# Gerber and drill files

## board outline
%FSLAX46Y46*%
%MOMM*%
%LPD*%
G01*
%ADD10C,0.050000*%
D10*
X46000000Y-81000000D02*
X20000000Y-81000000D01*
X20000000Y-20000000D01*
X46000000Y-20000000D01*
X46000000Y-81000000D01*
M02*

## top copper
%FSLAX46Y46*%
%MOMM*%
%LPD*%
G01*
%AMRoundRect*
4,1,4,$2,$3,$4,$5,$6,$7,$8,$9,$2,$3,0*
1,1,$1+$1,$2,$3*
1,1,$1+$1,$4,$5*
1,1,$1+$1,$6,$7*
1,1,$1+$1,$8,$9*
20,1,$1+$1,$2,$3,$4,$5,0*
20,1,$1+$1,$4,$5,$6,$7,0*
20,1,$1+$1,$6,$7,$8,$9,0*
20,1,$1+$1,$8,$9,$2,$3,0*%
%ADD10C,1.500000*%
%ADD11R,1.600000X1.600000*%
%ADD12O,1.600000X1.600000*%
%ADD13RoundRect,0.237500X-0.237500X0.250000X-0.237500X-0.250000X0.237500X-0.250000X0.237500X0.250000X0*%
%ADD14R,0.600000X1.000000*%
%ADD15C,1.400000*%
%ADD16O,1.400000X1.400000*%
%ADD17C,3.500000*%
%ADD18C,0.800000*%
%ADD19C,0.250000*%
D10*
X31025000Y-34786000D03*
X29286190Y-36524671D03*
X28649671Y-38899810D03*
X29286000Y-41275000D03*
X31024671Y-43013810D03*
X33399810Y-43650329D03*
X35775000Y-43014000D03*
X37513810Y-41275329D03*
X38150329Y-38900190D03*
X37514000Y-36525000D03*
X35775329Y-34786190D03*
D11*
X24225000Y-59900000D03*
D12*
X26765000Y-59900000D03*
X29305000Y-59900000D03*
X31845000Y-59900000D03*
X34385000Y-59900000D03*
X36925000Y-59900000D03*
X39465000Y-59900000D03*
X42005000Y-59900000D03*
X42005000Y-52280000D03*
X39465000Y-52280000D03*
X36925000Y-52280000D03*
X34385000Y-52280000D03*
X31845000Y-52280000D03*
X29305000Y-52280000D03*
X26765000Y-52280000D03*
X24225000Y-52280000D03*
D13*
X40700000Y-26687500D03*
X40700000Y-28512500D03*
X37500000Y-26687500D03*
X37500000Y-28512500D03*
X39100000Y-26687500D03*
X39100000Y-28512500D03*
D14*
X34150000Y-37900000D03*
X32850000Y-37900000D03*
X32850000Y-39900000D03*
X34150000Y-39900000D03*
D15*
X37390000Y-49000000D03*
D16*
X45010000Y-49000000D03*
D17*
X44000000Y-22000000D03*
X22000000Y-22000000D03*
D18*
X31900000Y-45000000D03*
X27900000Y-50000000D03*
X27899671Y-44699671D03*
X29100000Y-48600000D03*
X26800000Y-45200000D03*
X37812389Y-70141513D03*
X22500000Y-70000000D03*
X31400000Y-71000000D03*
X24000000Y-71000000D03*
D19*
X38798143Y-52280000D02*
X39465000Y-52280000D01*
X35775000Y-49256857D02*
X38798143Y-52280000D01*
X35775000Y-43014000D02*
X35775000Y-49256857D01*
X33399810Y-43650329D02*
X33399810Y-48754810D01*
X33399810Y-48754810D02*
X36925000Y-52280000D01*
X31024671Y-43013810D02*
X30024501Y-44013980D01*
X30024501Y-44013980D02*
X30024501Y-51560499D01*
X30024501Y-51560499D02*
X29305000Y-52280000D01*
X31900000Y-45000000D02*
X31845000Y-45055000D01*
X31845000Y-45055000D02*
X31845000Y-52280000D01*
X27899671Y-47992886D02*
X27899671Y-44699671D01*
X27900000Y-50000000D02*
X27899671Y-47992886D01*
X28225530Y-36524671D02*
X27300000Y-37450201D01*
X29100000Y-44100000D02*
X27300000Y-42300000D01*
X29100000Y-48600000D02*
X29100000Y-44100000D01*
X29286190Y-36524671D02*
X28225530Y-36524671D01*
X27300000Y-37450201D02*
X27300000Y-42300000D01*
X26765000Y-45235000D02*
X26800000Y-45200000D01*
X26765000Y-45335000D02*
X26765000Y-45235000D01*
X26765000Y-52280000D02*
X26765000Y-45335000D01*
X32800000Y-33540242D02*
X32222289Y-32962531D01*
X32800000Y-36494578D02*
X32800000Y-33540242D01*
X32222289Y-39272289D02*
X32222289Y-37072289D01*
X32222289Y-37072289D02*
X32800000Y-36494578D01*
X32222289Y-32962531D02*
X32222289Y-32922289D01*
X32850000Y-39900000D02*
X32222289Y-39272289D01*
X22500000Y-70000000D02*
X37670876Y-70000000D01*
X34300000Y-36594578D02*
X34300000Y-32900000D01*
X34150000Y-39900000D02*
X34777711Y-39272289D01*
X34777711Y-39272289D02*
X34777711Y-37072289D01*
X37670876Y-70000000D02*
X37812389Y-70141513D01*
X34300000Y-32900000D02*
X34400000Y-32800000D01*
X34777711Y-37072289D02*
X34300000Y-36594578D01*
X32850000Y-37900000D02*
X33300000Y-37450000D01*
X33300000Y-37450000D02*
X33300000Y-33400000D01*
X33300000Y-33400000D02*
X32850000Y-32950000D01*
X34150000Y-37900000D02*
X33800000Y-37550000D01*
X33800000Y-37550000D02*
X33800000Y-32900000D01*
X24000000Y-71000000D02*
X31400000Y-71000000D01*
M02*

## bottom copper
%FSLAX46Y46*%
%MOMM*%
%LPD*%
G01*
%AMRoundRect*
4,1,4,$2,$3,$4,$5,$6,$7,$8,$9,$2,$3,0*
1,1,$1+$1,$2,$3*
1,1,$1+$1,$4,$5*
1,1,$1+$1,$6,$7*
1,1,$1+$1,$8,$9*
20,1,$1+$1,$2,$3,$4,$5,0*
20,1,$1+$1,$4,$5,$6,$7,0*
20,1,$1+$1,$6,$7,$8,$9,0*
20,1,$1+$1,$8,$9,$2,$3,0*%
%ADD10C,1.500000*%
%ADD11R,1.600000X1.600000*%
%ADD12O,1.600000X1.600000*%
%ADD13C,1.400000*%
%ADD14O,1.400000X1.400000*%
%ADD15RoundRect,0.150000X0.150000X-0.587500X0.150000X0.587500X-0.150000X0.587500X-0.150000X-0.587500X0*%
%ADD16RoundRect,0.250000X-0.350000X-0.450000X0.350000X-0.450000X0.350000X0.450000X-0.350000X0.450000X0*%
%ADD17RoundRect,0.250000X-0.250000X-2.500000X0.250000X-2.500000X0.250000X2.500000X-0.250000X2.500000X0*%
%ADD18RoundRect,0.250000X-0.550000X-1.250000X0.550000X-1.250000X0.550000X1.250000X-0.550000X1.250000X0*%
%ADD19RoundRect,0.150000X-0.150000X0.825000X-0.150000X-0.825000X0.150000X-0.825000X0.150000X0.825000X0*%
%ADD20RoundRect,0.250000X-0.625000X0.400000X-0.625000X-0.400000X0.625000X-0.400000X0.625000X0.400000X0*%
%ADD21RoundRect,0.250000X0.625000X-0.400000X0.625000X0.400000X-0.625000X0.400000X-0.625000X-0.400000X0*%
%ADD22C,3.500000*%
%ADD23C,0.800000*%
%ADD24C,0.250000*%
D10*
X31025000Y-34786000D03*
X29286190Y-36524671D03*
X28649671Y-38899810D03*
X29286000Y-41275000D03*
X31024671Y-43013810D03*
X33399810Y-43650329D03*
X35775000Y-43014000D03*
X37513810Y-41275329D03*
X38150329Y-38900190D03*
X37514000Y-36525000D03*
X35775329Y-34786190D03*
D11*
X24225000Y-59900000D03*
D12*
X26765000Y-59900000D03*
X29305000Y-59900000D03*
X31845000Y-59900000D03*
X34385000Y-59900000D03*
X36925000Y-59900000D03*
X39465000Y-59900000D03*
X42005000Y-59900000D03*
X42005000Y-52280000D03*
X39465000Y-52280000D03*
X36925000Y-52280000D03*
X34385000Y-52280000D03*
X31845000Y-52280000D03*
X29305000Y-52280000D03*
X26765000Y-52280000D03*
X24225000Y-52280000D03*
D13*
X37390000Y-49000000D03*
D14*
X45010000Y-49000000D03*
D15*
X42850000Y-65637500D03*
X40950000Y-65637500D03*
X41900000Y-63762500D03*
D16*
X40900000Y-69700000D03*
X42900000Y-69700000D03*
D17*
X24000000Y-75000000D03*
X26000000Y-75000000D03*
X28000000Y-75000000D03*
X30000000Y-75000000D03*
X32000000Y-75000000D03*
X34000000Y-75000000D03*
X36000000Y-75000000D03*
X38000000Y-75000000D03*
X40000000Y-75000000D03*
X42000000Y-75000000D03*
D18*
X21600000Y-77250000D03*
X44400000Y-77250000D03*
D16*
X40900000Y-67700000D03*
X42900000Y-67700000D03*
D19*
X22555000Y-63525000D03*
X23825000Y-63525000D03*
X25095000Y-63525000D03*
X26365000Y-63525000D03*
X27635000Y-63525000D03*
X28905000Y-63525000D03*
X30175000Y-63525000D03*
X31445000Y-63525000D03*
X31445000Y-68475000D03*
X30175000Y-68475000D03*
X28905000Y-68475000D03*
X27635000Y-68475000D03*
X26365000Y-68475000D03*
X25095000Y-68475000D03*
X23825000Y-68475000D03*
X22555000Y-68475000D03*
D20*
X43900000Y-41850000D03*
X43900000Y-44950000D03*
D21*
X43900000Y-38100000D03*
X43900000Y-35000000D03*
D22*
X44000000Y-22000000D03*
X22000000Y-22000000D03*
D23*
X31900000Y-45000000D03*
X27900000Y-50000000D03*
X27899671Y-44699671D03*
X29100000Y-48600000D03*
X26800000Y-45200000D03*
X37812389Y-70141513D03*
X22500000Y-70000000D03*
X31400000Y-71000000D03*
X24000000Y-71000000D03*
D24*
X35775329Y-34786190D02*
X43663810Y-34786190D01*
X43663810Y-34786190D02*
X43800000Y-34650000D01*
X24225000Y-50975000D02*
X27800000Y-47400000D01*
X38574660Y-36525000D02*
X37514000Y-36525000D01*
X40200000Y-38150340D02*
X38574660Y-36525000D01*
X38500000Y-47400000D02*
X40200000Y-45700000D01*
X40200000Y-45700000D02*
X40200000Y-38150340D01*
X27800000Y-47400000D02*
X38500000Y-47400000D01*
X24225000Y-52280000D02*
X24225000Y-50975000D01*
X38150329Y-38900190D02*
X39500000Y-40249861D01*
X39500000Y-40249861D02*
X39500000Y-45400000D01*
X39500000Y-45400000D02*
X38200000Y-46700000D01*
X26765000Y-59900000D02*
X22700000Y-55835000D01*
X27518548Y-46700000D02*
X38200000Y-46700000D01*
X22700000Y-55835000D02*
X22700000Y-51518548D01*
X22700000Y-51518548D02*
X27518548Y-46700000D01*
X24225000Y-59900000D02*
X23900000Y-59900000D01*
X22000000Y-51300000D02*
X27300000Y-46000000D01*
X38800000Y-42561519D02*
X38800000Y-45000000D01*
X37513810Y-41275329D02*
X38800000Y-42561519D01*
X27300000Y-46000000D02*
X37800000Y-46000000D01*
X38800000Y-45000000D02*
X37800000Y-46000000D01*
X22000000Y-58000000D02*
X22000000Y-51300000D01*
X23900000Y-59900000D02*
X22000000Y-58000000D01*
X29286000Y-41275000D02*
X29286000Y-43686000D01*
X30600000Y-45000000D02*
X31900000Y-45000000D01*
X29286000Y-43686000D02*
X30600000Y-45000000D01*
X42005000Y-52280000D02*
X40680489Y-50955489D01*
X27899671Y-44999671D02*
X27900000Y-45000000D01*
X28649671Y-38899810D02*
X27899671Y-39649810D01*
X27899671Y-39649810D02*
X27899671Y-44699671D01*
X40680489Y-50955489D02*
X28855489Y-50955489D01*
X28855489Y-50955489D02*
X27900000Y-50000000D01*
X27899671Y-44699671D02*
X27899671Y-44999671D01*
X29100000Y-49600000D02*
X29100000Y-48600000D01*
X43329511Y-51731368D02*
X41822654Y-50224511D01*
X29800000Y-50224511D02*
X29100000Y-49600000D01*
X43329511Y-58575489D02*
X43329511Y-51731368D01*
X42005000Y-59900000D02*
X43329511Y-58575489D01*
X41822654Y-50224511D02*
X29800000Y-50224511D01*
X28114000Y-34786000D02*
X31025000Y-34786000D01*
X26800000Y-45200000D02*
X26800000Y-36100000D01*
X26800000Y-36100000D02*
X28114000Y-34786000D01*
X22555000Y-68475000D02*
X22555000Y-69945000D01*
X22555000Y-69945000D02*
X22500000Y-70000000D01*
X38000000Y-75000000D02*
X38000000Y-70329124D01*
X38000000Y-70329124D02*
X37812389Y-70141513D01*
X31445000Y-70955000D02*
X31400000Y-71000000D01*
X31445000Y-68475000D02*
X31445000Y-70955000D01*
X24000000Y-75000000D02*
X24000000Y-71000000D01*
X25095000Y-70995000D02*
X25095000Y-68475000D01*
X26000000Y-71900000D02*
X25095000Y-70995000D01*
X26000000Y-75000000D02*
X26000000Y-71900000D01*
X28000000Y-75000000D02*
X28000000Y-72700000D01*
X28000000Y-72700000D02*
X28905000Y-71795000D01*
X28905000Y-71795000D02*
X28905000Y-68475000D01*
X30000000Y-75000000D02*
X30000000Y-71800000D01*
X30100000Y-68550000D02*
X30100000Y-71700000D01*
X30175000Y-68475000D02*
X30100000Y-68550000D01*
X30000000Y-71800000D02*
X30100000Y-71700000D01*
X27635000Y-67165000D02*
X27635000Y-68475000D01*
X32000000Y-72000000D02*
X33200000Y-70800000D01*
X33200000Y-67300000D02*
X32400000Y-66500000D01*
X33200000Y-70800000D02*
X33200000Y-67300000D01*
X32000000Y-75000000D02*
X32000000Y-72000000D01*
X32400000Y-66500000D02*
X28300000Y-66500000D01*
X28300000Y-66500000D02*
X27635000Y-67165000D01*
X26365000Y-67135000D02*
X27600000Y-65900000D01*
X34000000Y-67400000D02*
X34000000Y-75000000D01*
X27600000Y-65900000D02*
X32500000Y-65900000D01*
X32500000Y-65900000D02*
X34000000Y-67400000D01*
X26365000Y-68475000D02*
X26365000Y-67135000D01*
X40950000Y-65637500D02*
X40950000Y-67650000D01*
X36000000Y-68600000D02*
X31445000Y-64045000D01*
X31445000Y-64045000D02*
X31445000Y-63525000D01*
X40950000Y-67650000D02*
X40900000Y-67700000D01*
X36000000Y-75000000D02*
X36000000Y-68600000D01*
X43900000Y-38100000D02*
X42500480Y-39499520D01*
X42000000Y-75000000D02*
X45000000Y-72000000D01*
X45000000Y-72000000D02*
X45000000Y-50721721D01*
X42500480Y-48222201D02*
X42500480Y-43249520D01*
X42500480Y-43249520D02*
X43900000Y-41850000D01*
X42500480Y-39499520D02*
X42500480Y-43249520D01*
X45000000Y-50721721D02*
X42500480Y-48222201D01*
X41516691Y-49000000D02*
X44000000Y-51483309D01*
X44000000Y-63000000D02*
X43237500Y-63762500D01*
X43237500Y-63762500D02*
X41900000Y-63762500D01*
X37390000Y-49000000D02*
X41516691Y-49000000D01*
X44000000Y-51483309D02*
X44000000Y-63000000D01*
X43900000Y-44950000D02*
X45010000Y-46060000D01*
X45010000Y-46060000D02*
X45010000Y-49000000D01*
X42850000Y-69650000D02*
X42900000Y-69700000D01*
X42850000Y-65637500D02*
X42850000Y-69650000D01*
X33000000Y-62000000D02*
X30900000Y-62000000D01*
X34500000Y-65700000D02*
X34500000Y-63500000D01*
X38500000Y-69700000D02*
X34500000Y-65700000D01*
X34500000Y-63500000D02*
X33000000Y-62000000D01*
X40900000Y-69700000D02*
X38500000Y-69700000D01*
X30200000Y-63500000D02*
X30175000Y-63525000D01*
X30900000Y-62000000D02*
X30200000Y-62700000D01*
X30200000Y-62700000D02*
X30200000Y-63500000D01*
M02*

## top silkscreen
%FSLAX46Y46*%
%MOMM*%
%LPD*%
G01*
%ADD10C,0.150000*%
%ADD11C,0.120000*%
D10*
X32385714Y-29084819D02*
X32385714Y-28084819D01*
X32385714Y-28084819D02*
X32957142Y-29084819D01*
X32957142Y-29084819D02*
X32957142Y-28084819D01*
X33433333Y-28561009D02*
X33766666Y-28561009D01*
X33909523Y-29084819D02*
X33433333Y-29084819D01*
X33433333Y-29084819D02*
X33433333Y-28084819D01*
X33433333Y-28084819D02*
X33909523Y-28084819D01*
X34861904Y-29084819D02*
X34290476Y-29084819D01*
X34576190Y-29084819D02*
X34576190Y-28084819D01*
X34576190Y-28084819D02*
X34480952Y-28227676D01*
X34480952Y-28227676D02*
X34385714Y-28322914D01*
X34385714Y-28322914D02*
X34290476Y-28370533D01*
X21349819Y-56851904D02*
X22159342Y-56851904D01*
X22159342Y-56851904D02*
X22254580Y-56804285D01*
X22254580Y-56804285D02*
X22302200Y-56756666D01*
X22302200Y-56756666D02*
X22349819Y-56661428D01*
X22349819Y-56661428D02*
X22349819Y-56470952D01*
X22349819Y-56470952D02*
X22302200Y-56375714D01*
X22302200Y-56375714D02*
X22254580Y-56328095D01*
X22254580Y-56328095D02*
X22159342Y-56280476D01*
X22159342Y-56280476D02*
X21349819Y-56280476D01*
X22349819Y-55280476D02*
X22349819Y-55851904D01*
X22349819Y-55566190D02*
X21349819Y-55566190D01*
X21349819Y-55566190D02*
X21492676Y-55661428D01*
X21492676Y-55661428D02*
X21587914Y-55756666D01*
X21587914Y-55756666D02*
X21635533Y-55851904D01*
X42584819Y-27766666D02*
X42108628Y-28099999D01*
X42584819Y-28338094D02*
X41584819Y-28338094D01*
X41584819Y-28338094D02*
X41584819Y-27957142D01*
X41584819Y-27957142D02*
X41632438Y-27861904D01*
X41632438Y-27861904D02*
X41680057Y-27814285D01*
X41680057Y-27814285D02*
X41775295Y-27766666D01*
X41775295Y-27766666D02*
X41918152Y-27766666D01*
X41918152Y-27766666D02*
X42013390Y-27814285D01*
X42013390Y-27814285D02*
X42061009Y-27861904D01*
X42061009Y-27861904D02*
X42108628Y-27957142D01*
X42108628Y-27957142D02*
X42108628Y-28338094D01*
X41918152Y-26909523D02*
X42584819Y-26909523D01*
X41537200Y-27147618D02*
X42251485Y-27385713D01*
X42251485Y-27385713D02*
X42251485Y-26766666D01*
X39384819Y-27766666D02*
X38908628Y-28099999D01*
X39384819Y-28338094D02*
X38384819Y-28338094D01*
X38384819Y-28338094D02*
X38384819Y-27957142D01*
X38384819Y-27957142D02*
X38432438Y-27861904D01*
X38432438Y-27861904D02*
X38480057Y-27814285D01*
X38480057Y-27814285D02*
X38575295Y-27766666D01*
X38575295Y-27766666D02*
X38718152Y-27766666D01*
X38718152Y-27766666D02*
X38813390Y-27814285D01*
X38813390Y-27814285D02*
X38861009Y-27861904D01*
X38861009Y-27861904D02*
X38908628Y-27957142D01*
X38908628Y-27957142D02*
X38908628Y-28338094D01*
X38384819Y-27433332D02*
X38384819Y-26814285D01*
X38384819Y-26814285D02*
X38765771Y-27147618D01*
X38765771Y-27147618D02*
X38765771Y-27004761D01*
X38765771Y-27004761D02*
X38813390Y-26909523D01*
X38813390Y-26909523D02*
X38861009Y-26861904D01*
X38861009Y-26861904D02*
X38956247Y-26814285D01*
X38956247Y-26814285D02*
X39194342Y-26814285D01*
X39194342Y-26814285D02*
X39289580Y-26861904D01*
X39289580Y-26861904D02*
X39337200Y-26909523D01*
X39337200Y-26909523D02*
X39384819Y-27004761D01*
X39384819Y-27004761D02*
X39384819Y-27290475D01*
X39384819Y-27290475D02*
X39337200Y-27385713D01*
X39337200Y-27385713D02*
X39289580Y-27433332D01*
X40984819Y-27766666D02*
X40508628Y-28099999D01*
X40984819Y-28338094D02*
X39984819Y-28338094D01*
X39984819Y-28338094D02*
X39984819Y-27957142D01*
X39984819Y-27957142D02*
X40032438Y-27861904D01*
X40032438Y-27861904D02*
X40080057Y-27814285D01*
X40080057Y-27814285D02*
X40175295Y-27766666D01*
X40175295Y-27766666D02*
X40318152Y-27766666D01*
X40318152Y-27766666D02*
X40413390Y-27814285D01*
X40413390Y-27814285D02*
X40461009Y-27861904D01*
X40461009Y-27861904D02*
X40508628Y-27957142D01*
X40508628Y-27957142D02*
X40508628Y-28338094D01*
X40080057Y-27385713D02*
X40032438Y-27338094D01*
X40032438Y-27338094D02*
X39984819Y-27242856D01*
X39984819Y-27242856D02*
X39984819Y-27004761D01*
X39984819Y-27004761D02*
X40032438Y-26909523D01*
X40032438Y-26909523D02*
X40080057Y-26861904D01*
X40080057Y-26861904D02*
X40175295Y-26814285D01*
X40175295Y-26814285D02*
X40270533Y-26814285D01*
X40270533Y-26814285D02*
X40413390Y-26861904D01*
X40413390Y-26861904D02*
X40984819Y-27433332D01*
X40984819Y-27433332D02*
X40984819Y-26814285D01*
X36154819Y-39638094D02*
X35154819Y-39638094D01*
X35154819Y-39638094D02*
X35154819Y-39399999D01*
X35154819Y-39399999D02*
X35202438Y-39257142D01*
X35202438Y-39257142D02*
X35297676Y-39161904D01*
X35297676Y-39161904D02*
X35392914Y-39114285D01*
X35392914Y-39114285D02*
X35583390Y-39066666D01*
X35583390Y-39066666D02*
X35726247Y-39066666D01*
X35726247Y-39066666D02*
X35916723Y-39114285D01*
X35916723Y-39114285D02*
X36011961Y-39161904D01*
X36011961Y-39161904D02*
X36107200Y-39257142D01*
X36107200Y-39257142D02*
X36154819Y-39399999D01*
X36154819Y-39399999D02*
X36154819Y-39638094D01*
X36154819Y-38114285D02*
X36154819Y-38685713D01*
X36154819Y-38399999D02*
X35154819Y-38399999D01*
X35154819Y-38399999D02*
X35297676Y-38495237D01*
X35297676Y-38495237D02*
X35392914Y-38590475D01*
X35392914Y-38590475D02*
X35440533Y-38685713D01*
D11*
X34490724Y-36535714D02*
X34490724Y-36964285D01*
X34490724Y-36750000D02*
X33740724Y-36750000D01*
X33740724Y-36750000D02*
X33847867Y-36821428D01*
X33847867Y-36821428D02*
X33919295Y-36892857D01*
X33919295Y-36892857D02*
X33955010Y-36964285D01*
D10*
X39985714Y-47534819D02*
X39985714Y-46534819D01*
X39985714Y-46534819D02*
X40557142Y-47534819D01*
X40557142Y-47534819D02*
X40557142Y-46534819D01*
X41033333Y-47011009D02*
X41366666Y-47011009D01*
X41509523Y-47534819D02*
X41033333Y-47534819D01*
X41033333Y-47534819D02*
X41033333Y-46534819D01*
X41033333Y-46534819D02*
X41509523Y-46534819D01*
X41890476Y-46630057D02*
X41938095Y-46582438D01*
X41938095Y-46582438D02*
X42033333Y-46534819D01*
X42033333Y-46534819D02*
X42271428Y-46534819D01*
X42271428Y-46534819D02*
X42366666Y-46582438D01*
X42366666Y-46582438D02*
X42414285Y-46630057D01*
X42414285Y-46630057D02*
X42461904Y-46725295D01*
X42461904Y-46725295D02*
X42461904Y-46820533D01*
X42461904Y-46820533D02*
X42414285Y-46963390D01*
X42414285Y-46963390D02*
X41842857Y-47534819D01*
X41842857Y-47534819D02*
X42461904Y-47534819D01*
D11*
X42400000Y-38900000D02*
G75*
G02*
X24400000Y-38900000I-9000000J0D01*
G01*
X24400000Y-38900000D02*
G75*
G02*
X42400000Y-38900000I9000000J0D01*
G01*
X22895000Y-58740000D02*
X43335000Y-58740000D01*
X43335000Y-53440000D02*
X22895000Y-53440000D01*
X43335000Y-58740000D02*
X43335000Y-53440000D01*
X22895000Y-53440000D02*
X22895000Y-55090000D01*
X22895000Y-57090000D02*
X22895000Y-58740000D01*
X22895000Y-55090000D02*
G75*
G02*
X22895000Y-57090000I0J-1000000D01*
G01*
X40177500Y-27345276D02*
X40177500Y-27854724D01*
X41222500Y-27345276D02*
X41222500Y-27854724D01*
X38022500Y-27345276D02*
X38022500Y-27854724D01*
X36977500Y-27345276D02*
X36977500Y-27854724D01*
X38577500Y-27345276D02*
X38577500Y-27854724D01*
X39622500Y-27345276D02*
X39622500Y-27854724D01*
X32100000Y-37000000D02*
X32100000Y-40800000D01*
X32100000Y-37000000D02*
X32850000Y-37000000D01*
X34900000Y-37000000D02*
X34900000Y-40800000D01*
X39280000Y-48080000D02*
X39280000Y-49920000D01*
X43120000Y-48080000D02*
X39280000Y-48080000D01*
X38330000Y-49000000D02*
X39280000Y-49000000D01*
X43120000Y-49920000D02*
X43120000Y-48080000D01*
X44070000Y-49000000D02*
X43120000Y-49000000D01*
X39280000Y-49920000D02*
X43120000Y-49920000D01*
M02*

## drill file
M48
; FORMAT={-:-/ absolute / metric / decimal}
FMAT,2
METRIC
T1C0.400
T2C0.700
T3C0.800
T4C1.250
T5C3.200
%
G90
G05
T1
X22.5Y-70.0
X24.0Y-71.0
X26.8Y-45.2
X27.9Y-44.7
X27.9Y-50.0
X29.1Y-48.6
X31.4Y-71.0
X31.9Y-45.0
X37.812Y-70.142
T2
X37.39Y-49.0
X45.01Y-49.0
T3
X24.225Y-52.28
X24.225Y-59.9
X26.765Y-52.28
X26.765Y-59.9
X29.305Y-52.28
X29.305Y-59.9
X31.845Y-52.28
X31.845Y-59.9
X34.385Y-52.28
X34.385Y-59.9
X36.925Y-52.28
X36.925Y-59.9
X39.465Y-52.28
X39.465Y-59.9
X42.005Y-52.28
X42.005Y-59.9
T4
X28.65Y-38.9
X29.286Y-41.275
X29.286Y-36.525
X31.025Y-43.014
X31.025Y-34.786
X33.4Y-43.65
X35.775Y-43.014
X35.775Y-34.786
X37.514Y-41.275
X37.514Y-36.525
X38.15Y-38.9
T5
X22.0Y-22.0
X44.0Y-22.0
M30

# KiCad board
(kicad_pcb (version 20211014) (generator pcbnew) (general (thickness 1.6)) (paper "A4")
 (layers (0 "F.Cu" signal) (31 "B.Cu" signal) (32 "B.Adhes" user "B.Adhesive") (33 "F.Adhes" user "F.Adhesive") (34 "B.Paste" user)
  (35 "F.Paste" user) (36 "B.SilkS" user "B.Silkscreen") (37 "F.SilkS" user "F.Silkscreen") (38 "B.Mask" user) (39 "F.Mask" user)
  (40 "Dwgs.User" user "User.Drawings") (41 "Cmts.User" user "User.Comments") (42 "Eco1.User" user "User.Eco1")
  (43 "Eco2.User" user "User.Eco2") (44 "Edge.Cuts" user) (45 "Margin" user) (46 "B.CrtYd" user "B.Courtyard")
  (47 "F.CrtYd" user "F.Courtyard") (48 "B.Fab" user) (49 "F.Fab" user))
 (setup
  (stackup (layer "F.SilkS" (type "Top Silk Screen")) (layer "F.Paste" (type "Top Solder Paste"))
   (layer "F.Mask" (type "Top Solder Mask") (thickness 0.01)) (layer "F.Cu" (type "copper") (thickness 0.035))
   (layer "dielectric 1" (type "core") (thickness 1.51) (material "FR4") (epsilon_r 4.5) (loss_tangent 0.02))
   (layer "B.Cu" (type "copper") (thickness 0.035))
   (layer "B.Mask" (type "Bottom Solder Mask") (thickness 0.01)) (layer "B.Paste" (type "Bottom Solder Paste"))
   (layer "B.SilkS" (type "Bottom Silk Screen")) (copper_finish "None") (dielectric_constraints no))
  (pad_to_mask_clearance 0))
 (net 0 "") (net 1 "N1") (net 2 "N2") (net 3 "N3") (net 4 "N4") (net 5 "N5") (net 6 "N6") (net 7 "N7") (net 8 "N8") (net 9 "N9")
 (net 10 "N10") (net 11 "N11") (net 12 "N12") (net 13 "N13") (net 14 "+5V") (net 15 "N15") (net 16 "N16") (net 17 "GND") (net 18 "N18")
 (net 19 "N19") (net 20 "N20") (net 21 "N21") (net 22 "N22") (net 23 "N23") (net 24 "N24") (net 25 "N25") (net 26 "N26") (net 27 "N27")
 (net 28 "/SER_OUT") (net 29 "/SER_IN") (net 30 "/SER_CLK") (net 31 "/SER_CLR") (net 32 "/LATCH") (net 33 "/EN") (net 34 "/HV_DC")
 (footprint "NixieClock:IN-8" (layer "F.Cu") (at 33.5 38.9)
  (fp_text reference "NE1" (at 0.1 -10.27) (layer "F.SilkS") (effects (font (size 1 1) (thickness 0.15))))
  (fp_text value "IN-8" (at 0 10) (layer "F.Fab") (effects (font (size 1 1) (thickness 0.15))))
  (fp_circle (center -0.1 0) (end -0.1 9) (layer "F.SilkS") (width 0.12) (fill none))
  (pad "1" thru_hole circle locked (at -2.475 -4.114) (size 1.5 1.5) (drill 1.25) (layers *.Cu *.Mask) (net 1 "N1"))
  (pad "2" thru_hole circle locked (at -4.21381 -2.375329) (size 1.5 1.5) (drill 1.25) (layers *.Cu *.Mask) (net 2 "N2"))
  (pad "3" thru_hole circle locked (at -4.850329 -0.00019) (size 1.5 1.5) (drill 1.25) (layers *.Cu *.Mask) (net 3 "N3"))
  (pad "4" thru_hole circle locked (at -4.214 2.375) (size 1.5 1.5) (drill 1.25) (layers *.Cu *.Mask) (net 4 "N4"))
  (pad "5" thru_hole circle locked (at -2.475329 4.11381) (size 1.5 1.5) (drill 1.25) (layers *.Cu *.Mask) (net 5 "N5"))
  (pad "6" thru_hole circle locked (at -0.10019 4.750329) (size 1.5 1.5) (drill 1.25) (layers *.Cu *.Mask) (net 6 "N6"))
  (pad "7" thru_hole circle locked (at 2.275 4.114) (size 1.5 1.5) (drill 1.25) (layers *.Cu *.Mask) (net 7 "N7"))
  (pad "8" thru_hole circle locked (at 4.01381 2.375329) (size 1.5 1.5) (drill 1.25) (layers *.Cu *.Mask) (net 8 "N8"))
  (pad "9" thru_hole circle locked (at 4.650329 0.00019) (size 1.5 1.5) (drill 1.25) (layers *.Cu *.Mask) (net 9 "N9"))
  (pad "10" thru_hole circle locked (at 4.014 -2.375) (size 1.5 1.5) (drill 1.25) (layers *.Cu *.Mask) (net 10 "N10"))
  (pad "11" thru_hole circle locked (at 2.275329 -4.11381) (size 1.5 1.5) (drill 1.25) (layers *.Cu *.Mask) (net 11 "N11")))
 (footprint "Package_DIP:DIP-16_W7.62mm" (layer "F.Cu") (at 24.225 59.9 90)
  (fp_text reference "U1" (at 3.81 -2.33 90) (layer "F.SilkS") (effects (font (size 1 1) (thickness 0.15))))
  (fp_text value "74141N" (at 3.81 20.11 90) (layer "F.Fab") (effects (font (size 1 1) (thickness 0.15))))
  (fp_line (start 1.16 -1.33) (end 1.16 19.11) (layer "F.SilkS") (width 0.12))
  (fp_line (start 6.46 19.11) (end 6.46 -1.33) (layer "F.SilkS") (width 0.12))
  (fp_line (start 1.16 19.11) (end 6.46 19.11) (layer "F.SilkS") (width 0.12))
  (fp_line (start 6.46 -1.33) (end 4.81 -1.33) (layer "F.SilkS") (width 0.12))
  (fp_line (start 2.81 -1.33) (end 1.16 -1.33) (layer "F.SilkS") (width 0.12))
  (fp_arc (start 4.81 -1.33) (mid 3.81 -0.33) (end 2.81 -1.33) (layer "F.SilkS") (width 0.12))
  (pad "1" thru_hole rect locked (at 0 0 90) (size 1.6 1.6) (drill 0.8) (layers *.Cu *.Mask) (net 8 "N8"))
  (pad "2" thru_hole oval locked (at 0 2.54 90) (size 1.6 1.6) (drill 0.8) (layers *.Cu *.Mask) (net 9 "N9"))
  (pad "3" thru_hole oval locked (at 0 5.08 90) (size 1.6 1.6) (drill 0.8) (layers *.Cu *.Mask) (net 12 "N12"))
  (pad "4" thru_hole oval locked (at 0 7.62 90) (size 1.6 1.6) (drill 0.8) (layers *.Cu *.Mask) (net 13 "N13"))
  (pad "5" thru_hole oval locked (at 0 10.16 90) (size 1.6 1.6) (drill 0.8) (layers *.Cu *.Mask) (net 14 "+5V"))
  (pad "6" thru_hole oval locked (at 0 12.7 90) (size 1.6 1.6) (drill 0.8) (layers *.Cu *.Mask) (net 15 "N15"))
  (pad "7" thru_hole oval locked (at 0 15.24 90) (size 1.6 1.6) (drill 0.8) (layers *.Cu *.Mask) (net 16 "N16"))
  (pad "8" thru_hole oval locked (at 0 17.78 90) (size 1.6 1.6) (drill 0.8) (layers *.Cu *.Mask) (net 2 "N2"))
  (pad "9" thru_hole oval locked (at 7.62 17.78 90) (size 1.6 1.6) (drill 0.8) (layers *.Cu *.Mask) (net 3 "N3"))
  (pad "10" thru_hole oval locked (at 7.62 15.24 90) (size 1.6 1.6) (drill 0.8) (layers *.Cu *.Mask) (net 7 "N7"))
  (pad "11" thru_hole oval locked (at 7.62 12.7 90) (size 1.6 1.6) (drill 0.8) (layers *.Cu *.Mask) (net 6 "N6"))
  (pad "12" thru_hole oval locked (at 7.62 10.16 90) (size 1.6 1.6) (drill 0.8) (layers *.Cu *.Mask) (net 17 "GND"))
  (pad "13" thru_hole oval locked (at 7.62 7.62 90) (size 1.6 1.6) (drill 0.8) (layers *.Cu *.Mask) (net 4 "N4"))
  (pad "14" thru_hole oval locked (at 7.62 5.08 90) (size 1.6 1.6) (drill 0.8) (layers *.Cu *.Mask) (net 5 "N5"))
  (pad "15" thru_hole oval locked (at 7.62 2.54 90) (size 1.6 1.6) (drill 0.8) (layers *.Cu *.Mask) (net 1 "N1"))
  (pad "16" thru_hole oval locked (at 7.62 0 90) (size 1.6 1.6) (drill 0.8) (layers *.Cu *.Mask) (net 10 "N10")))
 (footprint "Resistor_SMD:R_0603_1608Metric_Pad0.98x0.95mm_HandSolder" (layer "F.Cu") (at 40.7 27.6 -90)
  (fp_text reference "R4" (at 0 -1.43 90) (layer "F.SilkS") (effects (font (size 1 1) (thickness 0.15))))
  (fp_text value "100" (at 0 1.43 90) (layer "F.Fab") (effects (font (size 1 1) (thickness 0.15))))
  (fp_line (start -0.254724 0.5225) (end 0.254724 0.5225) (layer "F.SilkS") (width 0.12))
  (fp_line (start -0.254724 -0.5225) (end 0.254724 -0.5225) (layer "F.SilkS") (width 0.12))
  (pad "1" smd roundrect locked (at -0.9125 0 270) (size 0.975 0.95) (layers "F.Cu" "F.Paste" "F.Mask") (roundrect_rratio 0.25)
   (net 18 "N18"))
  (pad "2" smd roundrect locked (at 0.9125 0 270) (size 0.975 0.95) (layers "F.Cu" "F.Paste" "F.Mask") (roundrect_rratio 0.25)
   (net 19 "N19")))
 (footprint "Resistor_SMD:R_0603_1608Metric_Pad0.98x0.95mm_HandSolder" (layer "F.Cu") (at 37.5 27.6 -90)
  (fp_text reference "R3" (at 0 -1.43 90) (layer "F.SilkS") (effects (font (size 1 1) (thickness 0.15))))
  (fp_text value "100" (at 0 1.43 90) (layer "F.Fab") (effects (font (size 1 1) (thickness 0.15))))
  (fp_line (start -0.254724 -0.5225) (end 0.254724 -0.5225) (layer "F.SilkS") (width 0.12))
  (fp_line (start -0.254724 0.5225) (end 0.254724 0.5225) (layer "F.SilkS") (width 0.12))
  (pad "1" smd roundrect locked (at -0.9125 0 270) (size 0.975 0.95) (layers "F.Cu" "F.Paste" "F.Mask") (roundrect_rratio 0.25)
   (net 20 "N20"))
  (pad "2" smd roundrect locked (at 0.9125 0 270) (size 0.975 0.95) (layers "F.Cu" "F.Paste" "F.Mask") (roundrect_rratio 0.25)
   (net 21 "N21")))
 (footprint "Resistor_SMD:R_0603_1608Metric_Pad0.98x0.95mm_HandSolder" (layer "F.Cu") (at 39.1 27.6 -90)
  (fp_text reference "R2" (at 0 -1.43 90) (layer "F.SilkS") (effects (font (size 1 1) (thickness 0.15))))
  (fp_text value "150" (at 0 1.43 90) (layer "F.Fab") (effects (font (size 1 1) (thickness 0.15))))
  (fp_line (start -0.254724 0.5225) (end 0.254724 0.5225) (layer "F.SilkS") (width 0.12))
  (fp_line (start -0.254724 -0.5225) (end 0.254724 -0.5225) (layer "F.SilkS") (width 0.12))
  (pad "1" smd roundrect locked (at -0.9125 0 270) (size 0.975 0.95) (layers "F.Cu" "F.Paste" "F.Mask") (roundrect_rratio 0.25)
   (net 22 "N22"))
  (pad "2" smd roundrect locked (at 0.9125 0 270) (size 0.975 0.95) (layers "F.Cu" "F.Paste" "F.Mask") (roundrect_rratio 0.25)
   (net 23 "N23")))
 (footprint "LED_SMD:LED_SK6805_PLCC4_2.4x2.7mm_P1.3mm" (layer "F.Cu") (at 33.5 38.9 -90)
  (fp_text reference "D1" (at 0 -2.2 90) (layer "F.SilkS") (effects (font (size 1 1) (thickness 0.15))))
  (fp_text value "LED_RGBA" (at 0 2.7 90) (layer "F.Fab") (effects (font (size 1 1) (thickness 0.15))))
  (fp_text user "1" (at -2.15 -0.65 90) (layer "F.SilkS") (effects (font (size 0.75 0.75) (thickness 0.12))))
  (fp_line (start -1.9 1.4) (end 1.9 1.4) (layer "F.SilkS") (width 0.12))
  (fp_line (start -1.9 1.4) (end -1.9 0.65) (layer "F.SilkS") (width 0.12))
  (fp_line (start -1.9 -1.4) (end 1.9 -1.4) (layer "F.SilkS") (width 0.12))
  (pad "1" smd rect locked (at -1 -0.65 270) (size 1 0.6) (layers "F.Cu" "F.Paste" "F.Mask") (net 22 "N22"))
  (pad "2" smd rect locked (at -1 0.65 270) (size 1 0.6) (layers "F.Cu" "F.Paste" "F.Mask") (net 20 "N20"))
  (pad "3" smd rect locked (at 1 0.65 270) (size 1 0.6) (layers "F.Cu" "F.Paste" "F.Mask") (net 18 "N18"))
  (pad "4" smd rect locked (at 1 -0.65 270) (size 1 0.6) (layers "F.Cu" "F.Paste" "F.Mask") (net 14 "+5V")))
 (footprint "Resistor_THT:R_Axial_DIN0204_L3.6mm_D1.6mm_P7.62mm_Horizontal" (layer "F.Cu") (at 37.39 49)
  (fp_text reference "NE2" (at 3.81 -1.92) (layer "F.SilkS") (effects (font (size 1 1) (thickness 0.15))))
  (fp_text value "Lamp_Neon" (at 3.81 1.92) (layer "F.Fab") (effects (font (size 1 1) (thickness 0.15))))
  (fp_line (start 1.89 -0.92) (end 1.89 0.92) (layer "F.SilkS") (width 0.12))
  (fp_line (start 5.73 -0.92) (end 1.89 -0.92) (layer "F.SilkS") (width 0.12))
  (fp_line (start 0.94 0) (end 1.89 0) (layer "F.SilkS") (width 0.12))
  (fp_line (start 5.73 0.92) (end 5.73 -0.92) (layer "F.SilkS") (width 0.12))
  (fp_line (start 6.68 0) (end 5.73 0) (layer "F.SilkS") (width 0.12))
  (fp_line (start 1.89 0.92) (end 5.73 0.92) (layer "F.SilkS") (width 0.12))
  (pad "1" thru_hole circle locked (at 0 0) (size 1.4 1.4) (drill 0.7) (layers *.Cu *.Mask) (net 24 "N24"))
  (pad "2" thru_hole oval locked (at 7.62 0) (size 1.4 1.4) (drill 0.7) (layers *.Cu *.Mask) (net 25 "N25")))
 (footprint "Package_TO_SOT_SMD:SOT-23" (layer "B.Cu") (at 41.9 64.7 90)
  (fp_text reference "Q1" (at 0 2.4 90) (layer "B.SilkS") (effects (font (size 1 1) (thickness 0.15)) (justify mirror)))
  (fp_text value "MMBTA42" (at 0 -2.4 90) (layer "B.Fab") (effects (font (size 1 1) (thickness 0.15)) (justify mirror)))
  (pad "1" smd roundrect locked (at -0.9375 0.95 90) (size 1.475 0.6) (layers "B.Cu" "B.Paste" "B.Mask") (roundrect_rratio 0.25)
   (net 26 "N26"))
  (pad "2" smd roundrect locked (at -0.9375 -0.95 90) (size 1.475 0.6) (layers "B.Cu" "B.Paste" "B.Mask") (roundrect_rratio 0.25)
   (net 17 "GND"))
  (pad "3" smd roundrect locked (at 0.9375 0 90) (size 1.475 0.6) (layers "B.Cu" "B.Paste" "B.Mask") (roundrect_rratio 0.25) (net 24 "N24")))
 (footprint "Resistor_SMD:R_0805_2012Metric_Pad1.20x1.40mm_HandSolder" (layer "B.Cu") (at 41.9 69.7)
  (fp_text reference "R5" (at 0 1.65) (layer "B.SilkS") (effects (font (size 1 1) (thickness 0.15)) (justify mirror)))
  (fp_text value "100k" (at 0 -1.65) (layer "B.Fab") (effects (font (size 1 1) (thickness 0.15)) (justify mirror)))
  (pad "1" smd roundrect locked (at -1 0) (size 1.2 1.4) (layers "B.Cu" "B.Paste" "B.Mask") (roundrect_rratio 0.208333) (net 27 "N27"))
  (pad "2" smd roundrect locked (at 1 0) (size 1.2 1.4) (layers "B.Cu" "B.Paste" "B.Mask") (roundrect_rratio 0.208333) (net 26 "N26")))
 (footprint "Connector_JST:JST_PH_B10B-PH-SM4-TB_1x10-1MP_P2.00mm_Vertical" (layer "B.Cu") (at 33 75.5)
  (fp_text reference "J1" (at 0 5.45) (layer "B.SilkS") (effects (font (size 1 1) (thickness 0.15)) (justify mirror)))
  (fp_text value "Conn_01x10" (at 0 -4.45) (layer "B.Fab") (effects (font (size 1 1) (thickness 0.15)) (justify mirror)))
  (pad "1" smd roundrect locked (at -9 -0.5) (size 1 5.5) (layers "B.Cu" "B.Paste" "B.Mask") (roundrect_rratio 0.25) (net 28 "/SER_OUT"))
  (pad "2" smd roundrect locked (at -7 -0.5) (size 1 5.5) (layers "B.Cu" "B.Paste" "B.Mask") (roundrect_rratio 0.25) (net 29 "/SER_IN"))
  (pad "3" smd roundrect locked (at -5 -0.5) (size 1 5.5) (layers "B.Cu" "B.Paste" "B.Mask") (roundrect_rratio 0.25) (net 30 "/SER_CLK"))
  (pad "4" smd roundrect locked (at -3 -0.5) (size 1 5.5) (layers "B.Cu" "B.Paste" "B.Mask") (roundrect_rratio 0.25) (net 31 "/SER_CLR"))
  (pad "5" smd roundrect locked (at -1 -0.5) (size 1 5.5) (layers "B.Cu" "B.Paste" "B.Mask") (roundrect_rratio 0.25) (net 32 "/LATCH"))
  (pad "6" smd roundrect locked (at 1 -0.5) (size 1 5.5) (layers "B.Cu" "B.Paste" "B.Mask") (roundrect_rratio 0.25) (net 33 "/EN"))
  (pad "7" smd roundrect locked (at 3 -0.5) (size 1 5.5) (layers "B.Cu" "B.Paste" "B.Mask") (roundrect_rratio 0.25) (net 17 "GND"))
  (pad "8" smd roundrect locked (at 5 -0.5) (size 1 5.5) (layers "B.Cu" "B.Paste" "B.Mask") (roundrect_rratio 0.25) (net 14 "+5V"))
  (pad "9" smd roundrect locked (at 7 -0.5) (size 1 5.5) (layers "B.Cu" "B.Paste" "B.Mask") (roundrect_rratio 0.25) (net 17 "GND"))
  (pad "10" smd roundrect locked (at 9 -0.5) (size 1 5.5) (layers "B.Cu" "B.Paste" "B.Mask") (roundrect_rratio 0.25) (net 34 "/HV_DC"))
  (pad "MP" smd roundrect locked (at -11.4 1.75) (size 1.6 3) (layers "B.Cu" "B.Paste" "B.Mask") (roundrect_rratio 0.15625))
  (pad "MP" smd roundrect locked (at 11.4 1.75) (size 1.6 3) (layers "B.Cu" "B.Paste" "B.Mask") (roundrect_rratio 0.15625)))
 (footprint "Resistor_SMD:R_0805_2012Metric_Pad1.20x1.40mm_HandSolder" (layer "B.Cu") (at 41.9 67.7)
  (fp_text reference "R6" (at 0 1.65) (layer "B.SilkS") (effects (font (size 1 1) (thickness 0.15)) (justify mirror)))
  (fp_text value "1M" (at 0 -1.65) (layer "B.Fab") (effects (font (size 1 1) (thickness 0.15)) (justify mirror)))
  (pad "1" smd roundrect locked (at -1 0) (size 1.2 1.4) (layers "B.Cu" "B.Paste" "B.Mask") (roundrect_rratio 0.208333) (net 17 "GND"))
  (pad "2" smd roundrect locked (at 1 0) (size 1.2 1.4) (layers "B.Cu" "B.Paste" "B.Mask") (roundrect_rratio 0.208333) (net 26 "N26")))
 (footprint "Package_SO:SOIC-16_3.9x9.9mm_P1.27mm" (layer "B.Cu") (at 27 66 -90)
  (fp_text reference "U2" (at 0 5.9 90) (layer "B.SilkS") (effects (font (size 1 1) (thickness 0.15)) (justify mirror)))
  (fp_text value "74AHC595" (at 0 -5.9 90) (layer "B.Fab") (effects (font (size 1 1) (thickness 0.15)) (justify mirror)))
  (pad "1" smd roundrect locked (at -2.475 4.445 270) (size 1.95 0.6) (layers "B.Cu" "B.Paste" "B.Mask") (roundrect_rratio 0.25)
   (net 15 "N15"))
  (pad "2" smd roundrect locked (at -2.475 3.175 270) (size 1.95 0.6) (layers "B.Cu" "B.Paste" "B.Mask") (roundrect_rratio 0.25)
   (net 16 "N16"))
  (pad "3" smd roundrect locked (at -2.475 1.905 270) (size 1.95 0.6) (layers "B.Cu" "B.Paste" "B.Mask") (roundrect_rratio 0.25)
   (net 13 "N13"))
  (pad "4" smd roundrect locked (at -2.475 0.635 270) (size 1.95 0.6) (layers "B.Cu" "B.Paste" "B.Mask") (roundrect_rratio 0.25)
   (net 23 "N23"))
  (pad "5" smd roundrect locked (at -2.475 -0.635 270) (size 1.95 0.6) (layers "B.Cu" "B.Paste" "B.Mask") (roundrect_rratio 0.25)
   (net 21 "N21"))
  (pad "6" smd roundrect locked (at -2.475 -1.905 270) (size 1.95 0.6) (layers "B.Cu" "B.Paste" "B.Mask") (roundrect_rratio 0.25)
   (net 19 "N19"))
  (pad "7" smd roundrect locked (at -2.475 -3.175 270) (size 1.95 0.6) (layers "B.Cu" "B.Paste" "B.Mask") (roundrect_rratio 0.25)
   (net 27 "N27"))
  (pad "8" smd roundrect locked (at -2.475 -4.445 270) (size 1.95 0.6) (layers "B.Cu" "B.Paste" "B.Mask") (roundrect_rratio 0.25)
   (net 17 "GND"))
  (pad "9" smd roundrect locked (at 2.475 -4.445 270) (size 1.95 0.6) (layers "B.Cu" "B.Paste" "B.Mask") (roundrect_rratio 0.25)
   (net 28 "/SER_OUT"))
  (pad "10" smd roundrect locked (at 2.475 -3.175 270) (size 1.95 0.6) (layers "B.Cu" "B.Paste" "B.Mask") (roundrect_rratio 0.25)
   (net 31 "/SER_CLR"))
  (pad "11" smd roundrect locked (at 2.475 -1.905 270) (size 1.95 0.6) (layers "B.Cu" "B.Paste" "B.Mask") (roundrect_rratio 0.25)
   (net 30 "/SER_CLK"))
  (pad "12" smd roundrect locked (at 2.475 -0.635 270) (size 1.95 0.6) (layers "B.Cu" "B.Paste" "B.Mask") (roundrect_rratio 0.25)
   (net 32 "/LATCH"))
  (pad "13" smd roundrect locked (at 2.475 0.635 270) (size 1.95 0.6) (layers "B.Cu" "B.Paste" "B.Mask") (roundrect_rratio 0.25)
   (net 33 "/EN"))
  (pad "14" smd roundrect locked (at 2.475 1.905 270) (size 1.95 0.6) (layers "B.Cu" "B.Paste" "B.Mask") (roundrect_rratio 0.25)
   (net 29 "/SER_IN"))
  (pad "15" smd roundrect locked (at 2.475 3.175 270) (size 1.95 0.6) (layers "B.Cu" "B.Paste" "B.Mask") (roundrect_rratio 0.25)
   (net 12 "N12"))
  (pad "16" smd roundrect locked (at 2.475 4.445 270) (size 1.95 0.6) (layers "B.Cu" "B.Paste" "B.Mask") (roundrect_rratio 0.25)
   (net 14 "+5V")))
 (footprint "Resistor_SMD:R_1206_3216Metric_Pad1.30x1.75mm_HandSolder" (layer "B.Cu") (at 43.9 43.4 -90)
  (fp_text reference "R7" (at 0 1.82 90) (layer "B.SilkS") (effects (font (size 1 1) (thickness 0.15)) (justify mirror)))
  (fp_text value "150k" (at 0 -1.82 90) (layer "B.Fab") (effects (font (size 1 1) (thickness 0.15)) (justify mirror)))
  (pad "1" smd roundrect locked (at -1.55 0 270) (size 1.3 1.75) (layers "B.Cu" "B.Paste" "B.Mask") (roundrect_rratio 0.192308)
   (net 34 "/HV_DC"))
  (pad "2" smd roundrect locked (at 1.55 0 270) (size 1.3 1.75) (layers "B.Cu" "B.Paste" "B.Mask") (roundrect_rratio 0.192308)
   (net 25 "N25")))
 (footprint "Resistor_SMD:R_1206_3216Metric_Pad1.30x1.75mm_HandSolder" (layer "B.Cu") (at 43.9 36.55 90)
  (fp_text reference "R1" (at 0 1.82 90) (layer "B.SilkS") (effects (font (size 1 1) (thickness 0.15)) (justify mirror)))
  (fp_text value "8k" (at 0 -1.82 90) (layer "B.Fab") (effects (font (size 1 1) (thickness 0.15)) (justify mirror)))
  (pad "1" smd roundrect locked (at -1.55 0 90) (size 1.3 1.75) (layers "B.Cu" "B.Paste" "B.Mask") (roundrect_rratio 0.192308)
   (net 34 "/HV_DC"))
  (pad "2" smd roundrect locked (at 1.55 0 90) (size 1.3 1.75) (layers "B.Cu" "B.Paste" "B.Mask") (roundrect_rratio 0.192308) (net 11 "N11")))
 (gr_poly (pts (xy 46 81) (xy 20 81) (xy 20 20) (xy 46 20)) (layer "Edge.Cuts") (width 0.05) (fill none))
 (via (at 44 22) (size 3.5) (drill 3.2) (layers "F.Cu" "B.Cu") (free) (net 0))
 (via (at 22 22) (size 3.5) (drill 3.2) (layers "F.Cu" "B.Cu") (free) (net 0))
 (segment (start 35.775329 34.78619) (end 43.66381 34.78619) (width 0.25) (layer "B.Cu") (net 11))
 (segment (start 43.66381 34.78619) (end 43.8 34.65) (width 0.25) (layer "B.Cu") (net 11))
 (segment (start 24.225 50.975) (end 27.8 47.4) (width 0.25) (layer "B.Cu") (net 10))
 (segment (start 38.57466 36.525) (end 37.514 36.525) (width 0.25) (layer "B.Cu") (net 10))
 (segment (start 40.2 38.15034) (end 38.57466 36.525) (width 0.25) (layer "B.Cu") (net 10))
 (segment (start 38.5 47.4) (end 40.2 45.7) (width 0.25) (layer "B.Cu") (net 10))
 (segment (start 40.2 45.7) (end 40.2 38.15034) (width 0.25) (layer "B.Cu") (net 10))
 (segment (start 27.8 47.4) (end 38.5 47.4) (width 0.25) (layer "B.Cu") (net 10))
 (segment (start 24.225 52.28) (end 24.225 50.975) (width 0.25) (layer "B.Cu") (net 10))
 (segment (start 38.150329 38.90019) (end 39.5 40.249861) (width 0.25) (layer "B.Cu") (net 9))
 (segment (start 39.5 40.249861) (end 39.5 45.4) (width 0.25) (layer "B.Cu") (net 9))
 (segment (start 39.5 45.4) (end 38.2 46.7) (width 0.25) (layer "B.Cu") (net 9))
 (segment (start 26.765 59.9) (end 22.7 55.835) (width 0.25) (layer "B.Cu") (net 9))
 (segment (start 27.518548 46.7) (end 38.2 46.7) (width 0.25) (layer "B.Cu") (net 9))
 (segment (start 22.7 55.835) (end 22.7 51.518548) (width 0.25) (layer "B.Cu") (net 9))
 (segment (start 22.7 51.518548) (end 27.518548 46.7) (width 0.25) (layer "B.Cu") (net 9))
 (segment (start 24.225 59.9) (end 23.9 59.9) (width 0.25) (layer "B.Cu") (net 8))
 (segment (start 22 51.3) (end 27.3 46) (width 0.25) (layer "B.Cu") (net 8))
 (segment (start 38.8 42.561519) (end 38.8 45) (width 0.25) (layer "B.Cu") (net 8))
 (segment (start 37.51381 41.275329) (end 38.8 42.561519) (width 0.25) (layer "B.Cu") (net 8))
 (segment (start 27.3 46) (end 37.8 46) (width 0.25) (layer "B.Cu") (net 8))
 (segment (start 38.8 45) (end 37.8 46) (width 0.25) (layer "B.Cu") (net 8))
 (segment (start 22 58) (end 22 51.3) (width 0.25) (layer "B.Cu") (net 8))
 (segment (start 23.9 59.9) (end 22 58) (width 0.25) (layer "B.Cu") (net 8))
 (segment (start 38.798143 52.28) (end 39.465 52.28) (width 0.25) (layer "F.Cu") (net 7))
 (segment (start 35.775 49.256857) (end 38.798143 52.28) (width 0.25) (layer "F.Cu") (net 7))
 (segment (start 35.775 43.014) (end 35.775 49.256857) (width 0.25) (layer "F.Cu") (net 7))
 (segment (start 33.39981 43.650329) (end 33.39981 48.75481) (width 0.25) (layer "F.Cu") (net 6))
 (segment (start 33.39981 48.75481) (end 36.925 52.28) (width 0.25) (layer "F.Cu") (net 6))
 (segment (start 31.024671 43.01381) (end 30.024501 44.01398) (width 0.25) (layer "F.Cu") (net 5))
 (segment (start 30.024501 44.01398) (end 30.024501 51.560499) (width 0.25) (layer "F.Cu") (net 5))
 (segment (start 30.024501 51.560499) (end 29.305 52.28) (width 0.25) (layer "F.Cu") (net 5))
 (segment (start 31.9 45) (end 31.845 45.055) (width 0.25) (layer "F.Cu") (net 4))
 (segment (start 31.845 45.055) (end 31.845 52.28) (width 0.25) (layer "F.Cu") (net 4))
 (via (at 31.9 45) (size 0.8) (drill 0.4) (layers "F.Cu" "B.Cu") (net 4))
 (segment (start 29.286 41.275) (end 29.286 43.686) (width 0.25) (layer "B.Cu") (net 4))
 (segment (start 30.6 45) (end 31.9 45) (width 0.25) (layer "B.Cu") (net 4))
 (segment (start 29.286 43.686) (end 30.6 45) (width 0.25) (layer "B.Cu") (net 4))
 (segment (start 27.899671 47.992886) (end 27.899671 44.699671) (width 0.25) (layer "F.Cu") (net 3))
 (segment (start 27.9 50) (end 27.899671 47.992886) (width 0.25) (layer "F.Cu") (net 3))
 (via (at 27.9 50) (size 0.8) (drill 0.4) (layers "F.Cu" "B.Cu") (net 3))
 (via (at 27.899671 44.699671) (size 0.8) (drill 0.4) (layers "F.Cu" "B.Cu") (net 3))
 (segment (start 42.005 52.28) (end 40.680489 50.955489) (width 0.25) (layer "B.Cu") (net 3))
 (segment (start 27.899671 44.999671) (end 27.9 45) (width 0.25) (layer "B.Cu") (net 3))
 (segment (start 28.649671 38.89981) (end 27.899671 39.64981) (width 0.25) (layer "B.Cu") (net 3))
 (segment (start 27.899671 39.64981) (end 27.899671 44.699671) (width 0.25) (layer "B.Cu") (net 3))
 (segment (start 40.680489 50.955489) (end 28.855489 50.955489) (width 0.25) (layer "B.Cu") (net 3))
 (segment (start 28.855489 50.955489) (end 27.9 50) (width 0.25) (layer "B.Cu") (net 3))
 (segment (start 27.899671 44.699671) (end 27.899671 44.999671) (width 0.25) (layer "B.Cu") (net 3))
 (segment (start 28.22553 36.524671) (end 27.3 37.450201) (width 0.25) (layer "F.Cu") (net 2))
 (segment (start 29.1 44.1) (end 27.3 42.3) (width 0.25) (layer "F.Cu") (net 2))
 (segment (start 29.1 48.6) (end 29.1 44.1) (width 0.25) (layer "F.Cu") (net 2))
 (segment (start 29.28619 36.524671) (end 28.22553 36.524671) (width 0.25) (layer "F.Cu") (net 2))
 (segment (start 27.3 37.450201) (end 27.3 42.3) (width 0.25) (layer "F.Cu") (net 2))
 (via (at 29.1 48.6) (size 0.8) (drill 0.4) (layers "F.Cu" "B.Cu") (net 2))
 (segment (start 29.1 49.6) (end 29.1 48.6) (width 0.25) (layer "B.Cu") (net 2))
 (segment (start 43.329511 51.731368) (end 41.822654 50.224511) (width 0.25) (layer "B.Cu") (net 2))
 (segment (start 29.8 50.224511) (end 29.1 49.6) (width 0.25) (layer "B.Cu") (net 2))
 (segment (start 43.329511 58.575489) (end 43.329511 51.731368) (width 0.25) (layer "B.Cu") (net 2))
 (segment (start 42.005 59.9) (end 43.329511 58.575489) (width 0.25) (layer "B.Cu") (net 2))
 (segment (start 41.822654 50.224511) (end 29.8 50.224511) (width 0.25) (layer "B.Cu") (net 2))
 (segment (start 26.765 45.235) (end 26.8 45.2) (width 0.25) (layer "F.Cu") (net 1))
 (segment (start 26.765 45.335) (end 26.765 45.235) (width 0.25) (layer "F.Cu") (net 1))
 (segment (start 26.765 52.28) (end 26.765 45.335) (width 0.25) (layer "F.Cu") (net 1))
 (via (at 26.8 45.2) (size 0.8) (drill 0.4) (layers "F.Cu" "B.Cu") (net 1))
 (segment (start 28.114 34.786) (end 31.025 34.786) (width 0.25) (layer "B.Cu") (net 1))
 (segment (start 26.8 45.2) (end 26.8 36.1) (width 0.25) (layer "B.Cu") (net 1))
 (segment (start 26.8 36.1) (end 28.114 34.786) (width 0.25) (layer "B.Cu") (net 1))
 (segment (start 32.8 33.540242) (end 32.222289 32.962531) (width 0.25) (layer "F.Cu") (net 18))
 (segment (start 32.8 36.494578) (end 32.8 33.540242) (width 0.25) (layer "F.Cu") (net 18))
 (segment (start 32.222289 39.272289) (end 32.222289 37.072289) (width 0.25) (layer "F.Cu") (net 18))
 (segment (start 32.222289 37.072289) (end 32.8 36.494578) (width 0.25) (layer "F.Cu") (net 18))
 (segment (start 32.222289 32.962531) (end 32.222289 32.922289) (width 0.25) (layer "F.Cu") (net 18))
 (segment (start 32.85 39.9) (end 32.222289 39.272289) (width 0.25) (layer "F.Cu") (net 18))
 (segment (start 22.5 70) (end 37.670876 70) (width 0.25) (layer "F.Cu") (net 14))
 (segment (start 34.3 36.594578) (end 34.3 32.9) (width 0.25) (layer "F.Cu") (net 14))
 (segment (start 34.15 39.9) (end 34.777711 39.272289) (width 0.25) (layer "F.Cu") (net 14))
 (segment (start 34.777711 39.272289) (end 34.777711 37.072289) (width 0.25) (layer "F.Cu") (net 14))
 (segment (start 37.670876 70) (end 37.812389 70.141513) (width 0.25) (layer "F.Cu") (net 14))
 (segment (start 34.3 32.9) (end 34.4 32.8) (width 0.25) (layer "F.Cu") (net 14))
 (segment (start 34.777711 37.072289) (end 34.3 36.594578) (width 0.25) (layer "F.Cu") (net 14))
 (via (at 37.812389 70.141513) (size 0.8) (drill 0.4) (layers "F.Cu" "B.Cu") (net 14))
 (via (at 22.5 70) (size 0.8) (drill 0.4) (layers "F.Cu" "B.Cu") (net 14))
 (segment (start 22.555 68.475) (end 22.555 69.945) (width 0.25) (layer "B.Cu") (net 14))
 (segment (start 22.555 69.945) (end 22.5 70) (width 0.25) (layer "B.Cu") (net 14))
 (segment (start 38 75) (end 38 70.329124) (width 0.25) (layer "B.Cu") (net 14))
 (segment (start 38 70.329124) (end 37.812389 70.141513) (width 0.25) (layer "B.Cu") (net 14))
 (segment (start 32.85 37.9) (end 33.3 37.45) (width 0.25) (layer "F.Cu") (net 20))
 (segment (start 33.3 37.45) (end 33.3 33.4) (width 0.25) (layer "F.Cu") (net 20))
 (segment (start 33.3 33.4) (end 32.85 32.95) (width 0.25) (layer "F.Cu") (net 20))
 (segment (start 34.15 37.9) (end 33.8 37.55) (width 0.25) (layer "F.Cu") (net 22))
 (segment (start 33.8 37.55) (end 33.8 32.9) (width 0.25) (layer "F.Cu") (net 22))
 (segment (start 24 71) (end 31.4 71) (width 0.25) (layer "F.Cu") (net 28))
 (via (at 31.4 71) (size 0.8) (drill 0.4) (layers "F.Cu" "B.Cu") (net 28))
 (via (at 24 71) (size 0.8) (drill 0.4) (layers "F.Cu" "B.Cu") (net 28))
 (segment (start 31.445 70.955) (end 31.4 71) (width 0.25) (layer "B.Cu") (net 28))
 (segment (start 31.445 68.475) (end 31.445 70.955) (width 0.25) (layer "B.Cu") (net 28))
 (segment (start 24 75) (end 24 71) (width 0.25) (layer "B.Cu") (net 28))
 (segment (start 25.095 70.995) (end 25.095 68.475) (width 0.25) (layer "B.Cu") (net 29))
 (segment (start 26 71.9) (end 25.095 70.995) (width 0.25) (layer "B.Cu") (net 29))
 (segment (start 26 75) (end 26 71.9) (width 0.25) (layer "B.Cu") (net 29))
 (segment (start 28 75) (end 28 72.7) (width 0.25) (layer "B.Cu") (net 30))
 (segment (start 28 72.7) (end 28.905 71.795) (width 0.25) (layer "B.Cu") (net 30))
 (segment (start 28.905 71.795) (end 28.905 68.475) (width 0.25) (layer "B.Cu") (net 30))
 (segment (start 30 75) (end 30 71.8) (width 0.25) (layer "B.Cu") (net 31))
 (segment (start 30.1 68.55) (end 30.1 71.7) (width 0.25) (layer "B.Cu") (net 31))
 (segment (start 30.175 68.475) (end 30.1 68.55) (width 0.25) (layer "B.Cu") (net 31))
 (segment (start 30 71.8) (end 30.1 71.7) (width 0.25) (layer "B.Cu") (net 31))
 (segment (start 27.635 67.165) (end 27.635 68.475) (width 0.25) (layer "B.Cu") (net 32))
 (segment (start 32 72) (end 33.2 70.8) (width 0.25) (layer "B.Cu") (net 32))
 (segment (start 33.2 67.3) (end 32.4 66.5) (width 0.25) (layer "B.Cu") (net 32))
 (segment (start 33.2 70.8) (end 33.2 67.3) (width 0.25) (layer "B.Cu") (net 32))
 (segment (start 32 75) (end 32 72) (width 0.25) (layer "B.Cu") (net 32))
 (segment (start 32.4 66.5) (end 28.3 66.5) (width 0.25) (layer "B.Cu") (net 32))
 (segment (start 28.3 66.5) (end 27.635 67.165) (width 0.25) (layer "B.Cu") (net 32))
 (segment (start 26.365 67.135) (end 27.6 65.9) (width 0.25) (layer "B.Cu") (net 33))
 (segment (start 34 67.4) (end 34 75) (width 0.25) (layer "B.Cu") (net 33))
 (segment (start 27.6 65.9) (end 32.5 65.9) (width 0.25) (layer "B.Cu") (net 33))
 (segment (start 32.5 65.9) (end 34 67.4) (width 0.25) (layer "B.Cu") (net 33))
 (segment (start 26.365 68.475) (end 26.365 67.135) (width 0.25) (layer "B.Cu") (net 33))
 (segment (start 40.95 65.6375) (end 40.95 67.65) (width 0.25) (layer "B.Cu") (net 17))
 (segment (start 36 68.6) (end 31.445 64.045) (width 0.25) (layer "B.Cu") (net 17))
 (segment (start 31.445 64.045) (end 31.445 63.525) (width 0.25) (layer "B.Cu") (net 17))
 (segment (start 40.95 67.65) (end 40.9 67.7) (width 0.25) (layer "B.Cu") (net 17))
 (segment (start 36 75) (end 36 68.6) (width 0.25) (layer "B.Cu") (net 17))
 (segment (start 43.9 38.1) (end 42.50048 39.49952) (width 0.25) (layer "B.Cu") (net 34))
 (segment (start 42 75) (end 45 72) (width 0.25) (layer "B.Cu") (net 34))
 (segment (start 45 72) (end 45 50.721721) (width 0.25) (layer "B.Cu") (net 34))
 (segment (start 42.50048 48.222201) (end 42.50048 43.24952) (width 0.25) (layer "B.Cu") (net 34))
 (segment (start 42.50048 43.24952) (end 43.9 41.85) (width 0.25) (layer "B.Cu") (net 34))
 (segment (start 42.50048 39.49952) (end 42.50048 43.24952) (width 0.25) (layer "B.Cu") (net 34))
 (segment (start 45 50.721721) (end 42.50048 48.222201) (width 0.25) (layer "B.Cu") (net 34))
 (segment (start 41.516691 49) (end 44 51.483309) (width 0.25) (layer "B.Cu") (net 24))
 (segment (start 44 63) (end 43.2375 63.7625) (width 0.25) (layer "B.Cu") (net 24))
 (segment (start 43.2375 63.7625) (end 41.9 63.7625) (width 0.25) (layer "B.Cu") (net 24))
 (segment (start 37.39 49) (end 41.516691 49) (width 0.25) (layer "B.Cu") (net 24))
 (segment (start 44 51.483309) (end 44 63) (width 0.25) (layer "B.Cu") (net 24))
 (segment (start 43.9 44.95) (end 45.01 46.06) (width 0.25) (layer "B.Cu") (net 25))
 (segment (start 45.01 46.06) (end 45.01 49) (width 0.25) (layer "B.Cu") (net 25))
 (segment (start 42.85 69.65) (end 42.9 69.7) (width 0.25) (layer "B.Cu") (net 26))
 (segment (start 42.85 65.6375) (end 42.85 69.65) (width 0.25) (layer "B.Cu") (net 26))
 (segment (start 33 62) (end 30.9 62) (width 0.25) (layer "B.Cu") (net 27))
 (segment (start 34.5 65.7) (end 34.5 63.5) (width 0.25) (layer "B.Cu") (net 27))
 (segment (start 38.5 69.7) (end 34.5 65.7) (width 0.25) (layer "B.Cu") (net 27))
 (segment (start 34.5 63.5) (end 33 62) (width 0.25) (layer "B.Cu") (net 27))
 (segment (start 40.9 69.7) (end 38.5 69.7) (width 0.25) (layer "B.Cu") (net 27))
 (segment (start 30.2 63.5) (end 30.175 63.525) (width 0.25) (layer "B.Cu") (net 27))
 (segment (start 30.9 62) (end 30.2 62.7) (width 0.25) (layer "B.Cu") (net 27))
 (segment (start 30.2 62.7) (end 30.2 63.5) (width 0.25) (layer "B.Cu") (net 27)))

